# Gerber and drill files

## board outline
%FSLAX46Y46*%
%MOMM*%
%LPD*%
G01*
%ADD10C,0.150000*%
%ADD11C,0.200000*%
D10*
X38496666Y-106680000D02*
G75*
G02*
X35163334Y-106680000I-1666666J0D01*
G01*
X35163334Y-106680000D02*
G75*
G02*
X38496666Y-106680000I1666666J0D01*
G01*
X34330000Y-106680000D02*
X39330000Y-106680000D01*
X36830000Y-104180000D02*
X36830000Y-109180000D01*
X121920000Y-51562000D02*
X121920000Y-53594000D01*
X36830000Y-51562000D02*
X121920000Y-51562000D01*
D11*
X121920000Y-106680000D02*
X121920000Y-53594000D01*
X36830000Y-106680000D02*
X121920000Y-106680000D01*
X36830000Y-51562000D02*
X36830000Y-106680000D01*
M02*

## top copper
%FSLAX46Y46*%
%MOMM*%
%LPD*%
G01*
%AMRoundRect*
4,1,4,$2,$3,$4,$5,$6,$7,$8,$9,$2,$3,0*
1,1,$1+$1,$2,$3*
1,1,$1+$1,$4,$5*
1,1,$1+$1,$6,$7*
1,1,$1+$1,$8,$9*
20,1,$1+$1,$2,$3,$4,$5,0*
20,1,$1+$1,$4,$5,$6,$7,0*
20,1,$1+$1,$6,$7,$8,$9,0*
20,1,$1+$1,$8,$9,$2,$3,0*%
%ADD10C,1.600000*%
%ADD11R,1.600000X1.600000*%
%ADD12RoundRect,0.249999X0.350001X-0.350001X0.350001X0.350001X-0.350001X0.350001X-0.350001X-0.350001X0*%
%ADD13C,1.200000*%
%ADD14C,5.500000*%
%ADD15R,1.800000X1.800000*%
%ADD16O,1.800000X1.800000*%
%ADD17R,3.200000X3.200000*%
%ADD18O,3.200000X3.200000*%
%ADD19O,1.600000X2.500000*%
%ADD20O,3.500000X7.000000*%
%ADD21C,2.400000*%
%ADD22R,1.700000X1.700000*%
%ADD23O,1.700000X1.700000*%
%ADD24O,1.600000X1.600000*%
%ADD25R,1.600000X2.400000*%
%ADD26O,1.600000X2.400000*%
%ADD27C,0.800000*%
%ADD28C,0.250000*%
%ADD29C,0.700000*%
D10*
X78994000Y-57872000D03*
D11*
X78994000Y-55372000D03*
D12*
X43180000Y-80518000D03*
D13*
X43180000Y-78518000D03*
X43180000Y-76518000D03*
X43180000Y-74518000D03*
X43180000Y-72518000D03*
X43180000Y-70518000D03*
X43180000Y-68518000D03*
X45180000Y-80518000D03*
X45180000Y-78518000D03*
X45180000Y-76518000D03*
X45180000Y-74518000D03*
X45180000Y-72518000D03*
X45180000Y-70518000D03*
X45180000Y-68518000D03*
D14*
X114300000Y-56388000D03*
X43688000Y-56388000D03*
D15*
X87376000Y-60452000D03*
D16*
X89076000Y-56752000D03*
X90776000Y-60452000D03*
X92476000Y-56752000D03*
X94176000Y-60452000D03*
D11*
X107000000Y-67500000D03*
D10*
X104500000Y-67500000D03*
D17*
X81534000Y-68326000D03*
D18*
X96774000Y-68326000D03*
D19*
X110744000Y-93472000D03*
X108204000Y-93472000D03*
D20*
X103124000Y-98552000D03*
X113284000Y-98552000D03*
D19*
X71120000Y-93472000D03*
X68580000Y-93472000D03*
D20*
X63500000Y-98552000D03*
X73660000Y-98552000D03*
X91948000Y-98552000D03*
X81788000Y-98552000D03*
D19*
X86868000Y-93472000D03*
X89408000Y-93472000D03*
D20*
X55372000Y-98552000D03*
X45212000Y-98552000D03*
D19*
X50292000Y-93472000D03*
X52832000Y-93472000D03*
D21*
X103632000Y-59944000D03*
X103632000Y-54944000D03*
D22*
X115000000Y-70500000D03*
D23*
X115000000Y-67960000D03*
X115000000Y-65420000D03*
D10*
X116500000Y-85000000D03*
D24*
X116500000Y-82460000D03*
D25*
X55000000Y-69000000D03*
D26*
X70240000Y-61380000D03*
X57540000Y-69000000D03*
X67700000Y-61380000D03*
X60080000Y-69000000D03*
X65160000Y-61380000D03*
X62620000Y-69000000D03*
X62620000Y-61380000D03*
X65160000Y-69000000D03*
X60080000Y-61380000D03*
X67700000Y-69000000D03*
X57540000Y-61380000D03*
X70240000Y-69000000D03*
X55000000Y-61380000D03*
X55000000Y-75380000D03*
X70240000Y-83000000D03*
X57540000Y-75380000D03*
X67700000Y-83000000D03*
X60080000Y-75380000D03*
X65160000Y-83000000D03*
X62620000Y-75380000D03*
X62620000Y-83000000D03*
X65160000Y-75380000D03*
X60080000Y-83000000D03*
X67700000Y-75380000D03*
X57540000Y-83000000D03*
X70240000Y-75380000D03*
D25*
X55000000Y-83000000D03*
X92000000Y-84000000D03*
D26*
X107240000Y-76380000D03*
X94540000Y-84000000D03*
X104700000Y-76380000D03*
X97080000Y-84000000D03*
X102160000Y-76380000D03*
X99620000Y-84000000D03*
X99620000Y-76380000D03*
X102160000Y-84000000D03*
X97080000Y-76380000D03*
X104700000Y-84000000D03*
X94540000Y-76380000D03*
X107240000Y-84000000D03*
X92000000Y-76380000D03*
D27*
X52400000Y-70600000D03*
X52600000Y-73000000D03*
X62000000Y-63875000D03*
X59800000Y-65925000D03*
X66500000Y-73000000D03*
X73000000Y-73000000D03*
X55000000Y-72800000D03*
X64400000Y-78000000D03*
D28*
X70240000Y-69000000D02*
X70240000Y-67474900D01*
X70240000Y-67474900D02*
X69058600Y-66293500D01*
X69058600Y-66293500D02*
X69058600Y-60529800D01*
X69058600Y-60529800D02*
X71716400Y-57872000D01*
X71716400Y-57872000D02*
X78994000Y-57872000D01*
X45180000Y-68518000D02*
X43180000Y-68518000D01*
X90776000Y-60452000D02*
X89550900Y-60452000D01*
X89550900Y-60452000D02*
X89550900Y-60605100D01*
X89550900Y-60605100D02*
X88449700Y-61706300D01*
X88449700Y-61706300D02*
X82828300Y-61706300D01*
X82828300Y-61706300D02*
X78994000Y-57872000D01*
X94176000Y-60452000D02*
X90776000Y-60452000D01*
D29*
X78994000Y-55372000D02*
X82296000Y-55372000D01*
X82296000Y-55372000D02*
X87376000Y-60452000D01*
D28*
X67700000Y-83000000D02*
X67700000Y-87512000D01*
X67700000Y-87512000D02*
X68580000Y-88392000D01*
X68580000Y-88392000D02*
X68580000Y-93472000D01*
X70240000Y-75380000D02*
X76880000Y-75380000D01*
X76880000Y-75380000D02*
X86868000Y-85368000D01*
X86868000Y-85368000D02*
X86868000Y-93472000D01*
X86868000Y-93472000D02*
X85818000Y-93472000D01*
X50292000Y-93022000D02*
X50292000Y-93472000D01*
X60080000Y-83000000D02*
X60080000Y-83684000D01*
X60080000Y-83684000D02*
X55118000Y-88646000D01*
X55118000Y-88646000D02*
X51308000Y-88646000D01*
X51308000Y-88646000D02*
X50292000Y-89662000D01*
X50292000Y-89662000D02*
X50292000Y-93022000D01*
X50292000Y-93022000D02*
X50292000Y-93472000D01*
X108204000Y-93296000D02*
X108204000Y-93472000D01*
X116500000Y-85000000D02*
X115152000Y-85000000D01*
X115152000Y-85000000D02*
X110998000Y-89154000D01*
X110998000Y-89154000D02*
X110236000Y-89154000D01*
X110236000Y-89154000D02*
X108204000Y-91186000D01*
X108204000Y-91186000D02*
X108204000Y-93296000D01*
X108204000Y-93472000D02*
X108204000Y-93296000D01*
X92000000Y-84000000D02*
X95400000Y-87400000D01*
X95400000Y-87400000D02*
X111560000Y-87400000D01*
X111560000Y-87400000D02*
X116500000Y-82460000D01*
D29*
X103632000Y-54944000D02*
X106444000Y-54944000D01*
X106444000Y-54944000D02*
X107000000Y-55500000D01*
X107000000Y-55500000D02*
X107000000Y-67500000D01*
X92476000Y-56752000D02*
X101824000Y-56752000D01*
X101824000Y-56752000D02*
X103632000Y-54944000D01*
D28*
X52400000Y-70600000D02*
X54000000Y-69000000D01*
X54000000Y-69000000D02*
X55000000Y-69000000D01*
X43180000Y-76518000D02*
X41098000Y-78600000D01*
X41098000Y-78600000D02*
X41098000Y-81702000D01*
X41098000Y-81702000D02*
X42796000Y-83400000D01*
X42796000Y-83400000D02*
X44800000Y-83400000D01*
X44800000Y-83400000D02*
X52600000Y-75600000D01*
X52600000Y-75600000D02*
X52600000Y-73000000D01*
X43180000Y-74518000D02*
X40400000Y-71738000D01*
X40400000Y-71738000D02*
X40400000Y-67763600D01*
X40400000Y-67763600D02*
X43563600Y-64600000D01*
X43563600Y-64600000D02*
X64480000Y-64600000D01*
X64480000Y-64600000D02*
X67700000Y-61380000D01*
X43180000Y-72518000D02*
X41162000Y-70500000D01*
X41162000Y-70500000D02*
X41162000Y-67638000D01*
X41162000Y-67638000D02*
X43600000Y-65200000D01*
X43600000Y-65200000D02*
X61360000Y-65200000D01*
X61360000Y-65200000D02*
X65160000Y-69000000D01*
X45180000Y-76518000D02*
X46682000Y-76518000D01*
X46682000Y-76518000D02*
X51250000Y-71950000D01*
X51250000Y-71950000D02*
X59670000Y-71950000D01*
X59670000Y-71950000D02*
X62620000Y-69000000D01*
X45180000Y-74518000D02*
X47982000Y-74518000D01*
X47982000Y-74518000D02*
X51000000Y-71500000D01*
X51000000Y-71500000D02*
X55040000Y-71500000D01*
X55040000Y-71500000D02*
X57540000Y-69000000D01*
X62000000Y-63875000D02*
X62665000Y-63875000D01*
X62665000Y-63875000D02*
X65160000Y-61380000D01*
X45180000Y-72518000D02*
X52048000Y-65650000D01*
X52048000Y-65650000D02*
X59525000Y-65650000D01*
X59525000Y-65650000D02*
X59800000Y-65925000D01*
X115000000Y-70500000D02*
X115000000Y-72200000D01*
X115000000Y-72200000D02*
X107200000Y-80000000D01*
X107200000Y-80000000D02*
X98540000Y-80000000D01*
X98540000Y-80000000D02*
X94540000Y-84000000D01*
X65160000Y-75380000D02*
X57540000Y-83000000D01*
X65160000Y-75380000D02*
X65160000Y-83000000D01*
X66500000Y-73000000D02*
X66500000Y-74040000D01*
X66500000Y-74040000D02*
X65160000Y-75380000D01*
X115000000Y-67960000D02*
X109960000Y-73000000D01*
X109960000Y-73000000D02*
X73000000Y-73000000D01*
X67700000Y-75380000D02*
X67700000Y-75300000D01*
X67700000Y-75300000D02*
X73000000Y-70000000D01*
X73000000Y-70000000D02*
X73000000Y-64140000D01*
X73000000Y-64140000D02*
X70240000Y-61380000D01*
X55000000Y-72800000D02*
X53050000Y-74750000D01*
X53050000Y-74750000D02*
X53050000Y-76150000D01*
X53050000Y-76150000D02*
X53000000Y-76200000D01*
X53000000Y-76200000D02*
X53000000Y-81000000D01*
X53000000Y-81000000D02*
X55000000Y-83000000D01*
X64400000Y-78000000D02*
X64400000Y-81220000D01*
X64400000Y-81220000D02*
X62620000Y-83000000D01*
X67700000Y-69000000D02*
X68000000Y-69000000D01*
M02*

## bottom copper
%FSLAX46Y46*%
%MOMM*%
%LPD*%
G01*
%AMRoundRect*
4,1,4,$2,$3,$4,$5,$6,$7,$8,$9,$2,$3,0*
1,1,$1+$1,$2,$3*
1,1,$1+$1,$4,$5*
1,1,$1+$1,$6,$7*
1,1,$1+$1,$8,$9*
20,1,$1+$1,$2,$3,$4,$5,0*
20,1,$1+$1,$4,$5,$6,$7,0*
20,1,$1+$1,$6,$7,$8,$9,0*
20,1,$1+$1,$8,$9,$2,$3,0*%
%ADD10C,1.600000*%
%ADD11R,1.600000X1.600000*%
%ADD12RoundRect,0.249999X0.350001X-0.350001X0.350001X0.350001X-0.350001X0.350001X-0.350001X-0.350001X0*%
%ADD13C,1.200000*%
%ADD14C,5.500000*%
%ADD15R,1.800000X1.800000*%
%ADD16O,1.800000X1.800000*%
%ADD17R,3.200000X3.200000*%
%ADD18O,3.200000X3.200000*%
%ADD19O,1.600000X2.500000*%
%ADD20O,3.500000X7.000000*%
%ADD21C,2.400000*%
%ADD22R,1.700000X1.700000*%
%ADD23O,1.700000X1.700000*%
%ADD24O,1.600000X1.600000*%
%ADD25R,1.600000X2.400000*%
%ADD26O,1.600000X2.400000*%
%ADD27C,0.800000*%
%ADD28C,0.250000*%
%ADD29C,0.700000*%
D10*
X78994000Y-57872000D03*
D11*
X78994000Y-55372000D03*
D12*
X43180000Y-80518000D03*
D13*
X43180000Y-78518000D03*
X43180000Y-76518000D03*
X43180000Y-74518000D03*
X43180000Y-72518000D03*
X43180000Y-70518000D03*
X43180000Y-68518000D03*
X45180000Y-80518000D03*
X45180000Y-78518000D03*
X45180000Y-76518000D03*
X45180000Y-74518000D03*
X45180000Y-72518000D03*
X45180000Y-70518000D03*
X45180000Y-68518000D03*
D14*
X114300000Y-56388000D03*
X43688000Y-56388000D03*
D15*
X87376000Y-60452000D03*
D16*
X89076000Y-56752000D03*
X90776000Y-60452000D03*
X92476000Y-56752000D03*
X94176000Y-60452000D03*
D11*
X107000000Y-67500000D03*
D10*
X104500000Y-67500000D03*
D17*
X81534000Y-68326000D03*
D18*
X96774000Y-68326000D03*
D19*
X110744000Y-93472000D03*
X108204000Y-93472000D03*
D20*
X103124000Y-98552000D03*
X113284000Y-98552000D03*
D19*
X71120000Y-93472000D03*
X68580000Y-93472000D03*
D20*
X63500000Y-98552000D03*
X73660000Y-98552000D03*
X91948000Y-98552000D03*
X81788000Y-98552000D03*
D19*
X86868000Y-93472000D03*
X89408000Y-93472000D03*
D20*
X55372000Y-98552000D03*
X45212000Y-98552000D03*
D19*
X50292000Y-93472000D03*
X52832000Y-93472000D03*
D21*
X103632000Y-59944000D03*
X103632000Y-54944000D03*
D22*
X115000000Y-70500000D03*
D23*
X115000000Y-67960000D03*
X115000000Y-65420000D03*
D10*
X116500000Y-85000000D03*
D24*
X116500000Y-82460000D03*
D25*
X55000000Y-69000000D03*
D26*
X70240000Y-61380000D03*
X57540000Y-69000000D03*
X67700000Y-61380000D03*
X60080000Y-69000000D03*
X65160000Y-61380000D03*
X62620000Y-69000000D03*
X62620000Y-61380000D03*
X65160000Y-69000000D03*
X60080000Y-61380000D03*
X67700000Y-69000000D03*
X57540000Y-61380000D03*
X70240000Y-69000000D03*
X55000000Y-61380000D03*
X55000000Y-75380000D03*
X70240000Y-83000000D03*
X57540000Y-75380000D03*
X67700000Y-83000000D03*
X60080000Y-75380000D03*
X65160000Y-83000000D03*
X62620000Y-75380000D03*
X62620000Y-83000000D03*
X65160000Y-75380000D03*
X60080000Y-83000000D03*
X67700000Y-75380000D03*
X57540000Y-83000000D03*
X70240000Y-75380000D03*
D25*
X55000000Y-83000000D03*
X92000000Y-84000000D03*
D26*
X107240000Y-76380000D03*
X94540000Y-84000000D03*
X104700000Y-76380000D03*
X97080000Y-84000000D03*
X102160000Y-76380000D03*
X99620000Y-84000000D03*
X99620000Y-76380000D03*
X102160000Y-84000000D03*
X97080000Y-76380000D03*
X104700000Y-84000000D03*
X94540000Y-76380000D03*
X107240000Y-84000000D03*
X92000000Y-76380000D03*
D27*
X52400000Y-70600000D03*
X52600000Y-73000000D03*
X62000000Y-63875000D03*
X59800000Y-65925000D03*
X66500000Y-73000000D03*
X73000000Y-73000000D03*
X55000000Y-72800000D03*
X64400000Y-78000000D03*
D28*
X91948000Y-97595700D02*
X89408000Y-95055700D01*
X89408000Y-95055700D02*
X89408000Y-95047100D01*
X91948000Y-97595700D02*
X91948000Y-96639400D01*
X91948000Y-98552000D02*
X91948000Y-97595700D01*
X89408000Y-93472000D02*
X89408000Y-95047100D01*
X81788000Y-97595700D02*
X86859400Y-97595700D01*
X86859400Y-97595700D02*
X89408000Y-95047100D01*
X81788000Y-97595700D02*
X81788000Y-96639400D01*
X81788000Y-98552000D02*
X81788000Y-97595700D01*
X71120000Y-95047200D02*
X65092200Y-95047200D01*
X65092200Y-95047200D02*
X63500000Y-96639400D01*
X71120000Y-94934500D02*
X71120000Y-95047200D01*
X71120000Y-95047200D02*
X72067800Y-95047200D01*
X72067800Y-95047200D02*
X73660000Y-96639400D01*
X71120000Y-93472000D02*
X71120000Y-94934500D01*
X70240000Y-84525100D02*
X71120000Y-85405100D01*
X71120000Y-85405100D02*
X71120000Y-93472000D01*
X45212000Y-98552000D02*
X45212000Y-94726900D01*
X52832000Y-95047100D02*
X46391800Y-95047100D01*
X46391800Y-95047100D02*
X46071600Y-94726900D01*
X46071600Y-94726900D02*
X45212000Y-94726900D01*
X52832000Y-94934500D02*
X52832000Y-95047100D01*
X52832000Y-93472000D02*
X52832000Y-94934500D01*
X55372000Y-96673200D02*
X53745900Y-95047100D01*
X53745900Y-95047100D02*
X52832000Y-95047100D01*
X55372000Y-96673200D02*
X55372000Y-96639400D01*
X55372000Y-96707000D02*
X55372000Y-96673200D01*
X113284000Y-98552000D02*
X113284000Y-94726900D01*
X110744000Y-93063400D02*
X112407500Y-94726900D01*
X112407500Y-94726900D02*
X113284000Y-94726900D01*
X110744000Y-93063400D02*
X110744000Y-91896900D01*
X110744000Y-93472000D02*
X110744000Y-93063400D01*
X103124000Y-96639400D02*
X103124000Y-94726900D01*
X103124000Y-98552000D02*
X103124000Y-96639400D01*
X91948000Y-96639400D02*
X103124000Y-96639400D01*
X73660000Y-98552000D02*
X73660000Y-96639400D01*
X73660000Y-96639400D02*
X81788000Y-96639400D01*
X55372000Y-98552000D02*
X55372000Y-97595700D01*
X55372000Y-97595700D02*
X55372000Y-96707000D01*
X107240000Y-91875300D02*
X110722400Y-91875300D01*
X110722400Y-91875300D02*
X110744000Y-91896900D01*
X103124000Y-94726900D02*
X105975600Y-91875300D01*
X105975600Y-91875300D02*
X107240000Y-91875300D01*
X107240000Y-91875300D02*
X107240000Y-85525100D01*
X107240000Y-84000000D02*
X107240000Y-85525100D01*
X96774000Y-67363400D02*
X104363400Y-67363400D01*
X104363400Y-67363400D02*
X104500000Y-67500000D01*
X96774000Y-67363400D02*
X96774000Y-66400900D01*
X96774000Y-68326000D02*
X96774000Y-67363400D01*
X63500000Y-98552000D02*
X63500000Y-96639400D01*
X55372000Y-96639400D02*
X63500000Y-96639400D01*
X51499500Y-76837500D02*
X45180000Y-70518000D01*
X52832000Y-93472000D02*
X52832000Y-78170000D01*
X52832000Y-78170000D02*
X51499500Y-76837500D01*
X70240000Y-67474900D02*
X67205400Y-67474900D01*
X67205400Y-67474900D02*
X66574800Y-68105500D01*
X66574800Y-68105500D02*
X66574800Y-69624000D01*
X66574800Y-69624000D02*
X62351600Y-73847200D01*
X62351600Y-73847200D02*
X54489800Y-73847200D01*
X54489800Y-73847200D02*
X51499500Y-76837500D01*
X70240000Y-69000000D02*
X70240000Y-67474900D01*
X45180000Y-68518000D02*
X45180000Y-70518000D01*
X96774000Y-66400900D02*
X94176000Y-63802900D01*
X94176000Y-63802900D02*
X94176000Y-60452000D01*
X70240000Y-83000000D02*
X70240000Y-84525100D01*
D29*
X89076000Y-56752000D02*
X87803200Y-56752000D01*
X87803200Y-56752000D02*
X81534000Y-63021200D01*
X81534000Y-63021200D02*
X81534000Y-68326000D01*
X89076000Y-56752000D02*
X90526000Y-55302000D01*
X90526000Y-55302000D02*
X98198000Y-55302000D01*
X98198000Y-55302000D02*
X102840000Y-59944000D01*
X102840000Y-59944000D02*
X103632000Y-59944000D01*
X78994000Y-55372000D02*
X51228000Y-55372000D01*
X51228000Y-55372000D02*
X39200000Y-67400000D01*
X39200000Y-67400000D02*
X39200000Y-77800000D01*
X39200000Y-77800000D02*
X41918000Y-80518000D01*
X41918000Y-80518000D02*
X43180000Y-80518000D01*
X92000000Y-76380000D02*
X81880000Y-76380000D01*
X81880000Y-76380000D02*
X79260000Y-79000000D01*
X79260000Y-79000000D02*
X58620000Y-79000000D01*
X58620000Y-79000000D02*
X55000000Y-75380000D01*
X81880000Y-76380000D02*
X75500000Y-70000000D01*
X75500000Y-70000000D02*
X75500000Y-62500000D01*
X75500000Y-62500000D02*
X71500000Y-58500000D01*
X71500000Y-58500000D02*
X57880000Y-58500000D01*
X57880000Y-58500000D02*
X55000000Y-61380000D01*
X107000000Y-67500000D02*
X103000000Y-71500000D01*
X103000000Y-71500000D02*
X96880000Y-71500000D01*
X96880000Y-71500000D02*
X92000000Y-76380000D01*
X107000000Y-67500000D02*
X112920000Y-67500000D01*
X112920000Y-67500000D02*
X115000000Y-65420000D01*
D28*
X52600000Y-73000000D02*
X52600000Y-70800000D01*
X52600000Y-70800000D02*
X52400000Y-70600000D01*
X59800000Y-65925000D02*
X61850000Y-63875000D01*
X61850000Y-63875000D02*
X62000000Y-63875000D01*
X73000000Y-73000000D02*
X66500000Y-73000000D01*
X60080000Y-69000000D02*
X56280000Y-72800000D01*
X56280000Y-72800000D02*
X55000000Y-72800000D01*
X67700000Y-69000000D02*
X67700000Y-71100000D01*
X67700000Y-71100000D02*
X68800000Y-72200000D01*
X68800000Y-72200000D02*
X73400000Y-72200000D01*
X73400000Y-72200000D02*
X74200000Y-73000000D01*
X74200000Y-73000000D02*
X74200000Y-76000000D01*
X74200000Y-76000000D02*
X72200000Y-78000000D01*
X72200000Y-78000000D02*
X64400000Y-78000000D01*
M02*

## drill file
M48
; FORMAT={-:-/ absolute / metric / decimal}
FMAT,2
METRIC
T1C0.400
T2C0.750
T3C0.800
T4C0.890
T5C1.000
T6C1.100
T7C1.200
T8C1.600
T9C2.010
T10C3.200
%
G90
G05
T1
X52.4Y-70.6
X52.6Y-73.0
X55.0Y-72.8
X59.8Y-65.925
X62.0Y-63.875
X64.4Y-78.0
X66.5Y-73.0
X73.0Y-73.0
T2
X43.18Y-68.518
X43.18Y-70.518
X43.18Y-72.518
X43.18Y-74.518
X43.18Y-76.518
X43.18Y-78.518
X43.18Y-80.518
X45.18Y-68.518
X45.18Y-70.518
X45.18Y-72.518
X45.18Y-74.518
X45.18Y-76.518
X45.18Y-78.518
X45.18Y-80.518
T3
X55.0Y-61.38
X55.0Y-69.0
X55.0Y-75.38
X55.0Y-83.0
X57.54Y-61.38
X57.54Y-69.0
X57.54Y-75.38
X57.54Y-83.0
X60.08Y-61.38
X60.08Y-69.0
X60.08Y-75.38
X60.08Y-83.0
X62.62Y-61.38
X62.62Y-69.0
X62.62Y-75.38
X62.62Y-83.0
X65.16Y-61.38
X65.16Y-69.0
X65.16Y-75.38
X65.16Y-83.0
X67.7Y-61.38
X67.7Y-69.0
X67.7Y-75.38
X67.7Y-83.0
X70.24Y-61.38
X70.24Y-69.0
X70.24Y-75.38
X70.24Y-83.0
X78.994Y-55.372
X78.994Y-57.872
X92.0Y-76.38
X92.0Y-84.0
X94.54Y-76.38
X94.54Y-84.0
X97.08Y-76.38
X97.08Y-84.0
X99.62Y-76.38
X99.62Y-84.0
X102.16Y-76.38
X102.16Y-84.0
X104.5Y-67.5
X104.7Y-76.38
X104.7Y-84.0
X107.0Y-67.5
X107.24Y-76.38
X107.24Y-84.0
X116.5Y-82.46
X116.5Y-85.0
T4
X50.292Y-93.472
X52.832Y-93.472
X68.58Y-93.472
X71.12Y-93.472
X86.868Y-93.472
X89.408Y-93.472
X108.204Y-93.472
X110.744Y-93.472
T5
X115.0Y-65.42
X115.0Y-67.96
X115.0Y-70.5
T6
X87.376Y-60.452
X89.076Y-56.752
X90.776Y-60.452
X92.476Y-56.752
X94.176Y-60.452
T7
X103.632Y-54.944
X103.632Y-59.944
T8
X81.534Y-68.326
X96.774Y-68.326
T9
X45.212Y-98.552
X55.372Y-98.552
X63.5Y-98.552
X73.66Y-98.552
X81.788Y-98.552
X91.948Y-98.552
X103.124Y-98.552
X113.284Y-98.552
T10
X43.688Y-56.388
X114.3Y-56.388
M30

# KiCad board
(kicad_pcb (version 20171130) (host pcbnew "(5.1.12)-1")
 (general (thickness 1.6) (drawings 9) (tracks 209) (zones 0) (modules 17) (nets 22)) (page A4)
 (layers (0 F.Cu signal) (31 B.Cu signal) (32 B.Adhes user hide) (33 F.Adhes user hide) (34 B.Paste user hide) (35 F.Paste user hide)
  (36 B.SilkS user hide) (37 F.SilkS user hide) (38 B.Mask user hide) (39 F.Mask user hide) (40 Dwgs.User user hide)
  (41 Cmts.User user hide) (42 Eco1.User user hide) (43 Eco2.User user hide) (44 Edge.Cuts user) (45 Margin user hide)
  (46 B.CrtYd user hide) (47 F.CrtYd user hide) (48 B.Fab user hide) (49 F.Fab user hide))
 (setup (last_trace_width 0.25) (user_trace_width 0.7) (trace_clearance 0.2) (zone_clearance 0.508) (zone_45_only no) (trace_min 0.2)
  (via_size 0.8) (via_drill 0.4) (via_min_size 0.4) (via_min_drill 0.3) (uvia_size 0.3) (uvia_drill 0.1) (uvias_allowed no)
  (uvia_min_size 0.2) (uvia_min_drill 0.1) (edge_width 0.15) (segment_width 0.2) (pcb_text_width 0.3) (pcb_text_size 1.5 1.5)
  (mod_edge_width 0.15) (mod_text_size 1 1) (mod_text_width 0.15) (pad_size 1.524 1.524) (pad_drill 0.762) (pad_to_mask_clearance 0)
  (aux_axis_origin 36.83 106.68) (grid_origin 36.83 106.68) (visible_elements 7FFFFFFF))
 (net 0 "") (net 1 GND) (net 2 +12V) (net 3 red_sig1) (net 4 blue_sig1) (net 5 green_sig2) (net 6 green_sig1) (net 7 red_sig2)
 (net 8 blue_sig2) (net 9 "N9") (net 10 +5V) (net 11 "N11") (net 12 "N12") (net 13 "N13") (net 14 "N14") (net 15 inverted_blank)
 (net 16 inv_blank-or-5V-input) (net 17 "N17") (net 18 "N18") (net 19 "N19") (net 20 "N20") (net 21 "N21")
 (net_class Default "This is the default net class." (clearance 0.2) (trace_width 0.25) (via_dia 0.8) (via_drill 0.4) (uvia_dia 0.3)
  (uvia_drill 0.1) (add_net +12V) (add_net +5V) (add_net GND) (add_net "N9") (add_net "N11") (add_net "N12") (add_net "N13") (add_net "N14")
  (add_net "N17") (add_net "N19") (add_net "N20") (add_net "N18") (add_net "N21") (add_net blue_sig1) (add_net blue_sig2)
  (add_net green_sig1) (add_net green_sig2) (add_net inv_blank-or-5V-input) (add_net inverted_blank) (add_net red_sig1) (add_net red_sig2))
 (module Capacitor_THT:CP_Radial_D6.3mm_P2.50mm (layer F.Cu) (at 78.994 55.372 270)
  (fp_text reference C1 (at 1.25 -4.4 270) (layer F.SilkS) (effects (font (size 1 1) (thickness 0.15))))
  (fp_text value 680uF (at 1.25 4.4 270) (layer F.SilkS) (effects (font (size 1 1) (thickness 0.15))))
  (pad 2 thru_hole circle (at 2.5 0 270) (size 1.6 1.6) (drill 0.8) (layers *.Cu *.Mask) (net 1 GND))
  (pad 1 thru_hole rect (at 0 0 270) (size 1.6 1.6) (drill 0.8) (layers *.Cu *.Mask) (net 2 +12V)))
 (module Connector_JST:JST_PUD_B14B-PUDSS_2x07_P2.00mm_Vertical (layer F.Cu) (at 43.18 80.518 90)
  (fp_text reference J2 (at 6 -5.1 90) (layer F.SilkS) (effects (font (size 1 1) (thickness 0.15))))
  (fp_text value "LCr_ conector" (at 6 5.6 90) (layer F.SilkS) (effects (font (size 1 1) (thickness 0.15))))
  (pad 1 thru_hole roundrect (at 0 0 90) (size 1.2 1.2) (drill 0.75) (layers *.Cu *.Mask) (roundrect_rratio 0.2083325) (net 2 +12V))
  (pad 3 thru_hole circle (at 2 0 90) (size 1.2 1.2) (drill 0.75) (layers *.Cu *.Mask))
  (pad 5 thru_hole circle (at 4 0 90) (size 1.2 1.2) (drill 0.75) (layers *.Cu *.Mask) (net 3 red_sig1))
  (pad 7 thru_hole circle (at 6 0 90) (size 1.2 1.2) (drill 0.75) (layers *.Cu *.Mask) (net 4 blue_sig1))
  (pad 9 thru_hole circle (at 8 0 90) (size 1.2 1.2) (drill 0.75) (layers *.Cu *.Mask) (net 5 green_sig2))
  (pad 11 thru_hole circle (at 10 0 90) (size 1.2 1.2) (drill 0.75) (layers *.Cu *.Mask))
  (pad 13 thru_hole circle (at 12 0 90) (size 1.2 1.2) (drill 0.75) (layers *.Cu *.Mask) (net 1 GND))
  (pad 2 thru_hole circle (at 0 2 90) (size 1.2 1.2) (drill 0.75) (layers *.Cu *.Mask))
  (pad 4 thru_hole circle (at 2 2 90) (size 1.2 1.2) (drill 0.75) (layers *.Cu *.Mask))
  (pad 6 thru_hole circle (at 4 2 90) (size 1.2 1.2) (drill 0.75) (layers *.Cu *.Mask) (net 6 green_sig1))
  (pad 8 thru_hole circle (at 6 2 90) (size 1.2 1.2) (drill 0.75) (layers *.Cu *.Mask) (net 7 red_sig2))
  (pad 10 thru_hole circle (at 8 2 90) (size 1.2 1.2) (drill 0.75) (layers *.Cu *.Mask) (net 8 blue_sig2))
  (pad 12 thru_hole circle (at 10 2 90) (size 1.2 1.2) (drill 0.75) (layers *.Cu *.Mask) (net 1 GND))
  (pad 14 thru_hole circle (at 12 2 90) (size 1.2 1.2) (drill 0.75) (layers *.Cu *.Mask) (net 1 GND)))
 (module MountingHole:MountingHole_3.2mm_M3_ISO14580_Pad (layer F.Cu) (at 114.3 56.388)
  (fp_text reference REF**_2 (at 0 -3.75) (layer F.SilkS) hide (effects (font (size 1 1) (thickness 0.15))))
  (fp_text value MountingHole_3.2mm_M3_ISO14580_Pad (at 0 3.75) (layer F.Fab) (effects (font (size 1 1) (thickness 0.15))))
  (pad 1 thru_hole circle (at 0 0) (size 5.5 5.5) (drill 3.2) (layers *.Cu *.Mask)))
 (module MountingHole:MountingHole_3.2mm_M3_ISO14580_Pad (layer F.Cu) (at 43.688 56.388)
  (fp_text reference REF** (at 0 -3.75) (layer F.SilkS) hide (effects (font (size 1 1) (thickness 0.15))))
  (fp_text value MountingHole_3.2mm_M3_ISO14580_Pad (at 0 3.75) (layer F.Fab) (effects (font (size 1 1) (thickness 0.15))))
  (pad 1 thru_hole circle (at 0 0) (size 5.5 5.5) (drill 3.2) (layers *.Cu *.Mask)))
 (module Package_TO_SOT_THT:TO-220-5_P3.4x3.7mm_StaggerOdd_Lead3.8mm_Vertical (layer F.Cu) (at 87.376 60.452)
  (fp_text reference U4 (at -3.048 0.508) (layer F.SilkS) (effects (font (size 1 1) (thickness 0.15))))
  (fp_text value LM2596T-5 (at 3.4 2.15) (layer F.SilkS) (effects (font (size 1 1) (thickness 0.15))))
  (pad 1 thru_hole rect (at 0 0) (size 1.8 1.8) (drill 1.1) (layers *.Cu *.Mask) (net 2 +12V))
  (pad 2 thru_hole oval (at 1.7 -3.7) (size 1.8 1.8) (drill 1.1) (layers *.Cu *.Mask) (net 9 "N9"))
  (pad 3 thru_hole oval (at 3.4 0) (size 1.8 1.8) (drill 1.1) (layers *.Cu *.Mask) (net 1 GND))
  (pad 4 thru_hole oval (at 5.1 -3.7) (size 1.8 1.8) (drill 1.1) (layers *.Cu *.Mask) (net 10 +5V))
  (pad 5 thru_hole oval (at 6.8 0) (size 1.8 1.8) (drill 1.1) (layers *.Cu *.Mask) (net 1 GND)))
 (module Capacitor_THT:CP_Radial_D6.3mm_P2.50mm (layer F.Cu) (at 107 67.5 180)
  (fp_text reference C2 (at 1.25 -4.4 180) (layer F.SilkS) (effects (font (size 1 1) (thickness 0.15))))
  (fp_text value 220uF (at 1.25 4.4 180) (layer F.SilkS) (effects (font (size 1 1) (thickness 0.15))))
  (pad 1 thru_hole rect (at 0 0 180) (size 1.6 1.6) (drill 0.8) (layers *.Cu *.Mask) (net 10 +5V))
  (pad 2 thru_hole circle (at 2.5 0 180) (size 1.6 1.6) (drill 0.8) (layers *.Cu *.Mask) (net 1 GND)))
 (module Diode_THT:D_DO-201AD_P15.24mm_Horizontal (layer F.Cu) (at 81.534 68.326)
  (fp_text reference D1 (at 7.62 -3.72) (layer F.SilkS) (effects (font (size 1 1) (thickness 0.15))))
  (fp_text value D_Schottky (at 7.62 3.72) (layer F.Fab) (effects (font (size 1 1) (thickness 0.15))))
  (pad 1 thru_hole rect (at 0 0) (size 3.2 3.2) (drill 1.6) (layers *.Cu *.Mask) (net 9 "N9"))
  (pad 2 thru_hole oval (at 15.24 0) (size 3.2 3.2) (drill 1.6) (layers *.Cu *.Mask) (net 1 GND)))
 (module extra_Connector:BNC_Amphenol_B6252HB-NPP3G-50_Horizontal (layer F.Cu) (at 108.204 93.472 180)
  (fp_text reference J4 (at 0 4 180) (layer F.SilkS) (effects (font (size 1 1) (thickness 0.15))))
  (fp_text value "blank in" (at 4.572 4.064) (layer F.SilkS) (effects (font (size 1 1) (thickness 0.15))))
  (pad 2 thru_hole oval (at -2.54 0 180) (size 1.6 2.5) (drill 0.89) (layers *.Cu *.Mask) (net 1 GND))
  (pad 1 thru_hole oval (at 0 0 180) (size 1.6 2.5) (drill 0.89) (layers *.Cu *.Mask) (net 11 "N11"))
  (pad 2 thru_hole oval (at 5.08 -5.08 180) (size 3.5 7) (drill 2.01) (layers *.Cu *.Mask) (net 1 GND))
  (pad 2 thru_hole oval (at -5.08 -5.08 180) (size 3.5 7) (drill 2.01) (layers *.Cu *.Mask) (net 1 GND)))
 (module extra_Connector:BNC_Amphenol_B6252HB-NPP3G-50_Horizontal (layer F.Cu) (at 68.58 93.472 180)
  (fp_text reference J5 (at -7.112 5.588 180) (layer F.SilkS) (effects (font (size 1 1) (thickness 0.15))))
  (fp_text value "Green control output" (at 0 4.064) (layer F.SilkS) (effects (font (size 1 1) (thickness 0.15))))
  (pad 2 thru_hole oval (at -2.54 0 180) (size 1.6 2.5) (drill 0.89) (layers *.Cu *.Mask) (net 1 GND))
  (pad 1 thru_hole oval (at 0 0 180) (size 1.6 2.5) (drill 0.89) (layers *.Cu *.Mask) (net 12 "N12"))
  (pad 2 thru_hole oval (at 5.08 -5.08 180) (size 3.5 7) (drill 2.01) (layers *.Cu *.Mask) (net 1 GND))
  (pad 2 thru_hole oval (at -5.08 -5.08 180) (size 3.5 7) (drill 2.01) (layers *.Cu *.Mask) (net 1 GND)))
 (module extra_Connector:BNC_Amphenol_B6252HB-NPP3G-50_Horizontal (layer F.Cu) (at 86.868 93.472 180)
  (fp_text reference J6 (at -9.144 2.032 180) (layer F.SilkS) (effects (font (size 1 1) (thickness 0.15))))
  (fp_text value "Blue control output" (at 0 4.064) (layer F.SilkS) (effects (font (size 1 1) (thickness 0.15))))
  (pad 2 thru_hole oval (at -5.08 -5.08 180) (size 3.5 7) (drill 2.01) (layers *.Cu *.Mask) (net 1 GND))
  (pad 2 thru_hole oval (at 5.08 -5.08 180) (size 3.5 7) (drill 2.01) (layers *.Cu *.Mask) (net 1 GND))
  (pad 1 thru_hole oval (at 0 0 180) (size 1.6 2.5) (drill 0.89) (layers *.Cu *.Mask) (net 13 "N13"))
  (pad 2 thru_hole oval (at -2.54 0 180) (size 1.6 2.5) (drill 0.89) (layers *.Cu *.Mask) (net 1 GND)))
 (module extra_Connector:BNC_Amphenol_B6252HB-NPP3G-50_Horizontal (layer F.Cu) (at 50.292 93.472 180)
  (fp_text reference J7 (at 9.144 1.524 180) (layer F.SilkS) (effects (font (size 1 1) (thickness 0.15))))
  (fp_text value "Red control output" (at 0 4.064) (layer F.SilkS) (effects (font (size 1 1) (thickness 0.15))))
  (pad 2 thru_hole oval (at -5.08 -5.08 180) (size 3.5 7) (drill 2.01) (layers *.Cu *.Mask) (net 1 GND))
  (pad 2 thru_hole oval (at 5.08 -5.08 180) (size 3.5 7) (drill 2.01) (layers *.Cu *.Mask) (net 1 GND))
  (pad 1 thru_hole oval (at 0 0 180) (size 1.6 2.5) (drill 0.89) (layers *.Cu *.Mask) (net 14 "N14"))
  (pad 2 thru_hole oval (at -2.54 0 180) (size 1.6 2.5) (drill 0.89) (layers *.Cu *.Mask) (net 1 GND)))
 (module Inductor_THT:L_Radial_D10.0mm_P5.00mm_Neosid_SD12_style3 (layer F.Cu) (at 103.632 59.944 90)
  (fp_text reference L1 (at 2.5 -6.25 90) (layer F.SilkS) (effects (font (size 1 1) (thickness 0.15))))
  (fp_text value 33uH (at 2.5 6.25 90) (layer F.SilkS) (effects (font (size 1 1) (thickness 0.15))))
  (pad 1 thru_hole circle (at 0 0 90) (size 2.4 2.4) (drill 1.2) (layers *.Cu *.Mask) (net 9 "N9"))
  (pad 2 thru_hole circle (at 5 0 90) (size 2.4 2.4) (drill 1.2) (layers *.Cu *.Mask) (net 10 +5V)))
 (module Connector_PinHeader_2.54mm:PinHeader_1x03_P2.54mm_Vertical (layer F.Cu) (at 115 70.5 180)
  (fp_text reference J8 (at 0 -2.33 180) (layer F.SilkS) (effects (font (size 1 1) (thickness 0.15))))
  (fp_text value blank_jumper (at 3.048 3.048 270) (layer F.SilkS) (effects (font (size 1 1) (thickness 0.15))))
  (pad 1 thru_hole rect (at 0 0 180) (size 1.7 1.7) (drill 1) (layers *.Cu *.Mask) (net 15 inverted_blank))
  (pad 2 thru_hole oval (at 0 2.54 180) (size 1.7 1.7) (drill 1) (layers *.Cu *.Mask) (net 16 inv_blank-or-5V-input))
  (pad 3 thru_hole oval (at 0 5.08 180) (size 1.7 1.7) (drill 1) (layers *.Cu *.Mask) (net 10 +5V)))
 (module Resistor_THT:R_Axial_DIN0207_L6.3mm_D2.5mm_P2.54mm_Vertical (layer F.Cu) (at 116.5 85 90)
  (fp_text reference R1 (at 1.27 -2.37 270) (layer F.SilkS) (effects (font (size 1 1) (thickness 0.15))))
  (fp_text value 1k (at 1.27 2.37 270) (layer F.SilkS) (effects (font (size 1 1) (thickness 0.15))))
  (pad 1 thru_hole circle (at 0 0 90) (size 1.6 1.6) (drill 0.8) (layers *.Cu *.Mask) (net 11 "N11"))
  (pad 2 thru_hole oval (at 2.54 0 90) (size 1.6 1.6) (drill 0.8) (layers *.Cu *.Mask) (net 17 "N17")))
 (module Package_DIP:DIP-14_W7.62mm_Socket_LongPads (layer F.Cu) (at 55 69 90)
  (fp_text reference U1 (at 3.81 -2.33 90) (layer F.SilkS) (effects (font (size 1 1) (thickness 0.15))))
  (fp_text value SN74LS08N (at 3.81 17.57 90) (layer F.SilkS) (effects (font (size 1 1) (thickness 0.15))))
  (pad 1 thru_hole rect (at 0 0 90) (size 2.4 1.6) (drill 0.8) (layers *.Cu *.Mask) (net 3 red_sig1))
  (pad 8 thru_hole oval (at 7.62 15.24 90) (size 2.4 1.6) (drill 0.8) (layers *.Cu *.Mask) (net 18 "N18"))
  (pad 2 thru_hole oval (at 0 2.54 90) (size 2.4 1.6) (drill 0.8) (layers *.Cu *.Mask) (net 7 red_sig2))
  (pad 9 thru_hole oval (at 7.62 12.7 90) (size 2.4 1.6) (drill 0.8) (layers *.Cu *.Mask) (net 4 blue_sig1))
  (pad 3 thru_hole oval (at 0 5.08 90) (size 2.4 1.6) (drill 0.8) (layers *.Cu *.Mask) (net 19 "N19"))
  (pad 10 thru_hole oval (at 7.62 10.16 90) (size 2.4 1.6) (drill 0.8) (layers *.Cu *.Mask) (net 8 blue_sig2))
  (pad 4 thru_hole oval (at 0 7.62 90) (size 2.4 1.6) (drill 0.8) (layers *.Cu *.Mask) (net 6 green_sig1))
  (pad 11 thru_hole oval (at 7.62 7.62 90) (size 2.4 1.6) (drill 0.8) (layers *.Cu *.Mask))
  (pad 5 thru_hole oval (at 0 10.16 90) (size 2.4 1.6) (drill 0.8) (layers *.Cu *.Mask) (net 5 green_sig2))
  (pad 12 thru_hole oval (at 7.62 5.08 90) (size 2.4 1.6) (drill 0.8) (layers *.Cu *.Mask))
  (pad 6 thru_hole oval (at 0 12.7 90) (size 2.4 1.6) (drill 0.8) (layers *.Cu *.Mask) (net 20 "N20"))
  (pad 13 thru_hole oval (at 7.62 2.54 90) (size 2.4 1.6) (drill 0.8) (layers *.Cu *.Mask))
  (pad 7 thru_hole oval (at 0 15.24 90) (size 2.4 1.6) (drill 0.8) (layers *.Cu *.Mask) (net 1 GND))
  (pad 14 thru_hole oval (at 7.62 0 90) (size 2.4 1.6) (drill 0.8) (layers *.Cu *.Mask) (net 10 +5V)))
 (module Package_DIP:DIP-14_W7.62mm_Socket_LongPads (layer F.Cu) (at 55 83 90)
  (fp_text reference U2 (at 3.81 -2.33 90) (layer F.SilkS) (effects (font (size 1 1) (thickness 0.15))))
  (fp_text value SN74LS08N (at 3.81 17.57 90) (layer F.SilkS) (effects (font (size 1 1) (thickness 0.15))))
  (pad 14 thru_hole oval (at 7.62 0 90) (size 2.4 1.6) (drill 0.8) (layers *.Cu *.Mask) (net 10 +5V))
  (pad 7 thru_hole oval (at 0 15.24 90) (size 2.4 1.6) (drill 0.8) (layers *.Cu *.Mask) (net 1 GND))
  (pad 13 thru_hole oval (at 7.62 2.54 90) (size 2.4 1.6) (drill 0.8) (layers *.Cu *.Mask))
  (pad 6 thru_hole oval (at 0 12.7 90) (size 2.4 1.6) (drill 0.8) (layers *.Cu *.Mask) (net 12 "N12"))
  (pad 12 thru_hole oval (at 7.62 5.08 90) (size 2.4 1.6) (drill 0.8) (layers *.Cu *.Mask))
  (pad 5 thru_hole oval (at 0 10.16 90) (size 2.4 1.6) (drill 0.8) (layers *.Cu *.Mask) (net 16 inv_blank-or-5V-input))
  (pad 11 thru_hole oval (at 7.62 7.62 90) (size 2.4 1.6) (drill 0.8) (layers *.Cu *.Mask))
  (pad 4 thru_hole oval (at 0 7.62 90) (size 2.4 1.6) (drill 0.8) (layers *.Cu *.Mask) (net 20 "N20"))
  (pad 10 thru_hole oval (at 7.62 10.16 90) (size 2.4 1.6) (drill 0.8) (layers *.Cu *.Mask) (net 16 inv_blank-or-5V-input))
  (pad 3 thru_hole oval (at 0 5.08 90) (size 2.4 1.6) (drill 0.8) (layers *.Cu *.Mask) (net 14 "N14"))
  (pad 9 thru_hole oval (at 7.62 12.7 90) (size 2.4 1.6) (drill 0.8) (layers *.Cu *.Mask) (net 18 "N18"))
  (pad 2 thru_hole oval (at 0 2.54 90) (size 2.4 1.6) (drill 0.8) (layers *.Cu *.Mask) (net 16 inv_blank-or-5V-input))
  (pad 8 thru_hole oval (at 7.62 15.24 90) (size 2.4 1.6) (drill 0.8) (layers *.Cu *.Mask) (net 13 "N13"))
  (pad 1 thru_hole rect (at 0 0 90) (size 2.4 1.6) (drill 0.8) (layers *.Cu *.Mask) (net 19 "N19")))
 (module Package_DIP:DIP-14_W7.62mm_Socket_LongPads (layer F.Cu) (at 92 84 90)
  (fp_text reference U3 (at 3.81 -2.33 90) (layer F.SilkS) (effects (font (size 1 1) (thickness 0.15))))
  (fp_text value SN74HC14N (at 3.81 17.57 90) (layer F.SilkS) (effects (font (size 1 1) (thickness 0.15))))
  (pad 1 thru_hole rect (at 0 0 90) (size 2.4 1.6) (drill 0.8) (layers *.Cu *.Mask) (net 17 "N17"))
  (pad 8 thru_hole oval (at 7.62 15.24 90) (size 2.4 1.6) (drill 0.8) (layers *.Cu *.Mask))
  (pad 2 thru_hole oval (at 0 2.54 90) (size 2.4 1.6) (drill 0.8) (layers *.Cu *.Mask) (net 15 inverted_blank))
  (pad 9 thru_hole oval (at 7.62 12.7 90) (size 2.4 1.6) (drill 0.8) (layers *.Cu *.Mask))
  (pad 3 thru_hole oval (at 0 5.08 90) (size 2.4 1.6) (drill 0.8) (layers *.Cu *.Mask))
  (pad 10 thru_hole oval (at 7.62 10.16 90) (size 2.4 1.6) (drill 0.8) (layers *.Cu *.Mask))
  (pad 4 thru_hole oval (at 0 7.62 90) (size 2.4 1.6) (drill 0.8) (layers *.Cu *.Mask) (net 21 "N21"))
  (pad 11 thru_hole oval (at 7.62 7.62 90) (size 2.4 1.6) (drill 0.8) (layers *.Cu *.Mask))
  (pad 5 thru_hole oval (at 0 10.16 90) (size 2.4 1.6) (drill 0.8) (layers *.Cu *.Mask))
  (pad 12 thru_hole oval (at 7.62 5.08 90) (size 2.4 1.6) (drill 0.8) (layers *.Cu *.Mask))
  (pad 6 thru_hole oval (at 0 12.7 90) (size 2.4 1.6) (drill 0.8) (layers *.Cu *.Mask))
  (pad 13 thru_hole oval (at 7.62 2.54 90) (size 2.4 1.6) (drill 0.8) (layers *.Cu *.Mask))
  (pad 7 thru_hole oval (at 0 15.24 90) (size 2.4 1.6) (drill 0.8) (layers *.Cu *.Mask) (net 1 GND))
  (pad 14 thru_hole oval (at 7.62 0 90) (size 2.4 1.6) (drill 0.8) (layers *.Cu *.Mask) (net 10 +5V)))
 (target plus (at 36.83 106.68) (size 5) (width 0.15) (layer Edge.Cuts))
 (gr_line (start 121.92 51.562) (end 121.92 53.594) (layer Edge.Cuts) (width 0.15))
 (gr_line (start 36.83 51.562) (end 121.92 51.562) (layer Edge.Cuts) (width 0.15))
 (gr_line (start 121.92 106.68) (end 121.92 53.594) (layer Edge.Cuts) (width 0.2))
 (gr_line (start 36.83 106.68) (end 121.92 106.68) (layer Edge.Cuts) (width 0.2))
 (gr_line (start 36.83 51.562) (end 36.83 106.68) (layer Edge.Cuts) (width 0.2))
 (segment (start 91.948 97.5957) (end 89.408 95.0557) (width 0.25) (layer B.Cu) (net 1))
 (segment (start 89.408 95.0557) (end 89.408 95.0471) (width 0.25) (layer B.Cu) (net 1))
 (segment (start 91.948 97.5957) (end 91.948 96.6394) (width 0.25) (layer B.Cu) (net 1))
 (segment (start 91.948 98.552) (end 91.948 97.5957) (width 0.25) (layer B.Cu) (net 1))
 (segment (start 89.408 93.472) (end 89.408 95.0471) (width 0.25) (layer B.Cu) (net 1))
 (segment (start 81.788 97.5957) (end 86.8594 97.5957) (width 0.25) (layer B.Cu) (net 1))
 (segment (start 86.8594 97.5957) (end 89.408 95.0471) (width 0.25) (layer B.Cu) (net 1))
 (segment (start 81.788 97.5957) (end 81.788 96.6394) (width 0.25) (layer B.Cu) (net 1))
 (segment (start 81.788 98.552) (end 81.788 97.5957) (width 0.25) (layer B.Cu) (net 1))
 (segment (start 70.24 69) (end 70.24 67.4749) (width 0.25) (layer F.Cu) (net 1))
 (segment (start 70.24 67.4749) (end 69.0586 66.2935) (width 0.25) (layer F.Cu) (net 1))
 (segment (start 69.0586 66.2935) (end 69.0586 60.5298) (width 0.25) (layer F.Cu) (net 1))
 (segment (start 69.0586 60.5298) (end 71.7164 57.872) (width 0.25) (layer F.Cu) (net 1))
 (segment (start 71.7164 57.872) (end 78.994 57.872) (width 0.25) (layer F.Cu) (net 1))
 (segment (start 71.12 95.0472) (end 65.0922 95.0472) (width 0.25) (layer B.Cu) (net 1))
 (segment (start 65.0922 95.0472) (end 63.5 96.6394) (width 0.25) (layer B.Cu) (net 1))
 (segment (start 71.12 94.9345) (end 71.12 95.0472) (width 0.25) (layer B.Cu) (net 1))
 (segment (start 71.12 95.0472) (end 72.0678 95.0472) (width 0.25) (layer B.Cu) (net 1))
 (segment (start 72.0678 95.0472) (end 73.66 96.6394) (width 0.25) (layer B.Cu) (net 1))
 (segment (start 71.12 93.472) (end 71.12 94.9345) (width 0.25) (layer B.Cu) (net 1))
 (segment (start 70.24 84.5251) (end 71.12 85.4051) (width 0.25) (layer B.Cu) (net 1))
 (segment (start 71.12 85.4051) (end 71.12 93.472) (width 0.25) (layer B.Cu) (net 1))
 (segment (start 45.212 98.552) (end 45.212 94.7269) (width 0.25) (layer B.Cu) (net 1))
 (segment (start 52.832 95.0471) (end 46.3918 95.0471) (width 0.25) (layer B.Cu) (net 1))
 (segment (start 46.3918 95.0471) (end 46.0716 94.7269) (width 0.25) (layer B.Cu) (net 1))
 (segment (start 46.0716 94.7269) (end 45.212 94.7269) (width 0.25) (layer B.Cu) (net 1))
 (segment (start 52.832 94.9345) (end 52.832 95.0471) (width 0.25) (layer B.Cu) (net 1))
 (segment (start 52.832 93.472) (end 52.832 94.9345) (width 0.25) (layer B.Cu) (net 1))
 (segment (start 55.372 96.6732) (end 53.7459 95.0471) (width 0.25) (layer B.Cu) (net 1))
 (segment (start 53.7459 95.0471) (end 52.832 95.0471) (width 0.25) (layer B.Cu) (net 1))
 (segment (start 55.372 96.6732) (end 55.372 96.6394) (width 0.25) (layer B.Cu) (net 1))
 (segment (start 55.372 96.707) (end 55.372 96.6732) (width 0.25) (layer B.Cu) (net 1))
 (segment (start 113.284 98.552) (end 113.284 94.7269) (width 0.25) (layer B.Cu) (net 1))
 (segment (start 110.744 93.0634) (end 112.4075 94.7269) (width 0.25) (layer B.Cu) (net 1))
 (segment (start 112.4075 94.7269) (end 113.284 94.7269) (width 0.25) (layer B.Cu) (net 1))
 (segment (start 110.744 93.0634) (end 110.744 91.8969) (width 0.25) (layer B.Cu) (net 1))
 (segment (start 110.744 93.472) (end 110.744 93.0634) (width 0.25) (layer B.Cu) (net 1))
 (segment (start 103.124 96.6394) (end 103.124 94.7269) (width 0.25) (layer B.Cu) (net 1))
 (segment (start 103.124 98.552) (end 103.124 96.6394) (width 0.25) (layer B.Cu) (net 1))
 (segment (start 91.948 96.6394) (end 103.124 96.6394) (width 0.25) (layer B.Cu) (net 1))
 (segment (start 73.66 98.552) (end 73.66 96.6394) (width 0.25) (layer B.Cu) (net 1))
 (segment (start 73.66 96.6394) (end 81.788 96.6394) (width 0.25) (layer B.Cu) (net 1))
 (segment (start 55.372 98.552) (end 55.372 97.5957) (width 0.25) (layer B.Cu) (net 1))
 (segment (start 55.372 97.5957) (end 55.372 96.707) (width 0.25) (layer B.Cu) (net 1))
 (segment (start 107.24 91.8753) (end 110.7224 91.8753) (width 0.25) (layer B.Cu) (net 1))
 (segment (start 110.7224 91.8753) (end 110.744 91.8969) (width 0.25) (layer B.Cu) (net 1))
 (segment (start 103.124 94.7269) (end 105.9756 91.8753) (width 0.25) (layer B.Cu) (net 1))
 (segment (start 105.9756 91.8753) (end 107.24 91.8753) (width 0.25) (layer B.Cu) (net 1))
 (segment (start 107.24 91.8753) (end 107.24 85.5251) (width 0.25) (layer B.Cu) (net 1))
 (segment (start 107.24 84) (end 107.24 85.5251) (width 0.25) (layer B.Cu) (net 1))
 (segment (start 96.774 67.3634) (end 104.3634 67.3634) (width 0.25) (layer B.Cu) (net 1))
 (segment (start 104.3634 67.3634) (end 104.5 67.5) (width 0.25) (layer B.Cu) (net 1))
 (segment (start 96.774 67.3634) (end 96.774 66.4009) (width 0.25) (layer B.Cu) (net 1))
 (segment (start 96.774 68.326) (end 96.774 67.3634) (width 0.25) (layer B.Cu) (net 1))
 (segment (start 63.5 98.552) (end 63.5 96.6394) (width 0.25) (layer B.Cu) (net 1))
 (segment (start 55.372 96.6394) (end 63.5 96.6394) (width 0.25) (layer B.Cu) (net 1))
 (segment (start 51.4995 76.8375) (end 45.18 70.518) (width 0.25) (layer B.Cu) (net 1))
 (segment (start 52.832 93.472) (end 52.832 78.17) (width 0.25) (layer B.Cu) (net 1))
 (segment (start 52.832 78.17) (end 51.4995 76.8375) (width 0.25) (layer B.Cu) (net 1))
 (segment (start 70.24 67.4749) (end 67.2054 67.4749) (width 0.25) (layer B.Cu) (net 1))
 (segment (start 67.2054 67.4749) (end 66.5748 68.1055) (width 0.25) (layer B.Cu) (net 1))
 (segment (start 66.5748 68.1055) (end 66.5748 69.624) (width 0.25) (layer B.Cu) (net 1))
 (segment (start 66.5748 69.624) (end 62.3516 73.8472) (width 0.25) (layer B.Cu) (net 1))
 (segment (start 62.3516 73.8472) (end 54.4898 73.8472) (width 0.25) (layer B.Cu) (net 1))
 (segment (start 54.4898 73.8472) (end 51.4995 76.8375) (width 0.25) (layer B.Cu) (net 1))
 (segment (start 70.24 69) (end 70.24 67.4749) (width 0.25) (layer B.Cu) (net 1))
 (segment (start 45.18 68.518) (end 43.18 68.518) (width 0.25) (layer F.Cu) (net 1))
 (segment (start 45.18 68.518) (end 45.18 70.518) (width 0.25) (layer B.Cu) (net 1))
 (segment (start 90.776 60.452) (end 89.5509 60.452) (width 0.25) (layer F.Cu) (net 1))
 (segment (start 89.5509 60.452) (end 89.5509 60.6051) (width 0.25) (layer F.Cu) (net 1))
 (segment (start 89.5509 60.6051) (end 88.4497 61.7063) (width 0.25) (layer F.Cu) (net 1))
 (segment (start 88.4497 61.7063) (end 82.8283 61.7063) (width 0.25) (layer F.Cu) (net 1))
 (segment (start 82.8283 61.7063) (end 78.994 57.872) (width 0.25) (layer F.Cu) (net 1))
 (segment (start 94.176 60.452) (end 90.776 60.452) (width 0.25) (layer F.Cu) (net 1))
 (segment (start 96.774 66.4009) (end 94.176 63.8029) (width 0.25) (layer B.Cu) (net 1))
 (segment (start 94.176 63.8029) (end 94.176 60.452) (width 0.25) (layer B.Cu) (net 1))
 (segment (start 70.24 83) (end 70.24 84.5251) (width 0.25) (layer B.Cu) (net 1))
 (segment (start 89.076 56.752) (end 87.8032 56.752) (width 0.7) (layer B.Cu) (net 9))
 (segment (start 87.8032 56.752) (end 81.534 63.0212) (width 0.7) (layer B.Cu) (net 9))
 (segment (start 81.534 63.0212) (end 81.534 68.326) (width 0.7) (layer B.Cu) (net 9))
 (segment (start 89.076 56.752) (end 90.526 55.302) (width 0.7) (layer B.Cu) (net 9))
 (segment (start 90.526 55.302) (end 98.198 55.302) (width 0.7) (layer B.Cu) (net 9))
 (segment (start 98.198 55.302) (end 102.84 59.944) (width 0.7) (layer B.Cu) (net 9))
 (segment (start 102.84 59.944) (end 103.632 59.944) (width 0.7) (layer B.Cu) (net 9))
 (segment (start 78.994 55.372) (end 51.228 55.372) (width 0.7) (layer B.Cu) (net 2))
 (segment (start 51.228 55.372) (end 39.2 67.4) (width 0.7) (layer B.Cu) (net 2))
 (segment (start 39.2 67.4) (end 39.2 77.8) (width 0.7) (layer B.Cu) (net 2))
 (segment (start 39.2 77.8) (end 41.918 80.518) (width 0.7) (layer B.Cu) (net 2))
 (segment (start 41.918 80.518) (end 43.18 80.518) (width 0.7) (layer B.Cu) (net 2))
 (segment (start 78.994 55.372) (end 82.296 55.372) (width 0.7) (layer F.Cu) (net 2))
 (segment (start 82.296 55.372) (end 87.376 60.452) (width 0.7) (layer F.Cu) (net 2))
 (segment (start 67.7 83) (end 67.7 87.512) (width 0.25) (layer F.Cu) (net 12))
 (segment (start 67.7 87.512) (end 68.58 88.392) (width 0.25) (layer F.Cu) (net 12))
 (segment (start 68.58 88.392) (end 68.58 93.472) (width 0.25) (layer F.Cu) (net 12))
 (segment (start 70.24 75.38) (end 76.88 75.38) (width 0.25) (layer F.Cu) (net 13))
 (segment (start 76.88 75.38) (end 86.868 85.368) (width 0.25) (layer F.Cu) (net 13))
 (segment (start 86.868 85.368) (end 86.868 93.472) (width 0.25) (layer F.Cu) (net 13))
 (segment (start 86.868 93.472) (end 85.818 93.472) (width 0.25) (layer F.Cu) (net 13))
 (segment (start 50.292 93.022) (end 50.292 93.472) (width 0.25) (layer F.Cu) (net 14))
 (segment (start 60.08 83) (end 60.08 83.684) (width 0.25) (layer F.Cu) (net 14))
 (segment (start 60.08 83.684) (end 55.118 88.646) (width 0.25) (layer F.Cu) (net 14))
 (segment (start 55.118 88.646) (end 51.308 88.646) (width 0.25) (layer F.Cu) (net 14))
 (segment (start 51.308 88.646) (end 50.292 89.662) (width 0.25) (layer F.Cu) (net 14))
 (segment (start 50.292 89.662) (end 50.292 93.022) (width 0.25) (layer F.Cu) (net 14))
 (segment (start 50.292 93.022) (end 50.292 93.472) (width 0.25) (layer F.Cu) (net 14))
 (segment (start 108.204 93.296) (end 108.204 93.472) (width 0.25) (layer F.Cu) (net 11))
 (segment (start 116.5 85) (end 115.152 85) (width 0.25) (layer F.Cu) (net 11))
 (segment (start 115.152 85) (end 110.998 89.154) (width 0.25) (layer F.Cu) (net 11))
 (segment (start 110.998 89.154) (end 110.236 89.154) (width 0.25) (layer F.Cu) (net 11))
 (segment (start 110.236 89.154) (end 108.204 91.186) (width 0.25) (layer F.Cu) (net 11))
 (segment (start 108.204 91.186) (end 108.204 93.296) (width 0.25) (layer F.Cu) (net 11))
 (segment (start 108.204 93.472) (end 108.204 93.296) (width 0.25) (layer F.Cu) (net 11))
 (segment (start 92 84) (end 95.4 87.4) (width 0.25) (layer F.Cu) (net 17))
 (segment (start 95.4 87.4) (end 111.56 87.4) (width 0.25) (layer F.Cu) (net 17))
 (segment (start 111.56 87.4) (end 116.5 82.46) (width 0.25) (layer F.Cu) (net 17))
 (segment (start 92 76.38) (end 81.88 76.38) (width 0.7) (layer B.Cu) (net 10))
 (segment (start 103.632 54.944) (end 106.444 54.944) (width 0.7) (layer F.Cu) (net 10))
 (segment (start 106.444 54.944) (end 107 55.5) (width 0.7) (layer F.Cu) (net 10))
 (segment (start 107 55.5) (end 107 67.5) (width 0.7) (layer F.Cu) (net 10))
 (segment (start 92.476 56.752) (end 101.824 56.752) (width 0.7) (layer F.Cu) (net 10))
 (segment (start 101.824 56.752) (end 103.632 54.944) (width 0.7) (layer F.Cu) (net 10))
 (segment (start 81.88 76.38) (end 79.26 79) (width 0.7) (layer B.Cu) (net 10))
 (segment (start 79.26 79) (end 58.62 79) (width 0.7) (layer B.Cu) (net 10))
 (segment (start 58.62 79) (end 55 75.38) (width 0.7) (layer B.Cu) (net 10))
 (segment (start 81.88 76.38) (end 75.5 70) (width 0.7) (layer B.Cu) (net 10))
 (segment (start 75.5 70) (end 75.5 62.5) (width 0.7) (layer B.Cu) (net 10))
 (segment (start 75.5 62.5) (end 71.5 58.5) (width 0.7) (layer B.Cu) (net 10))
 (segment (start 71.5 58.5) (end 57.88 58.5) (width 0.7) (layer B.Cu) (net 10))
 (segment (start 57.88 58.5) (end 55 61.38) (width 0.7) (layer B.Cu) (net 10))
 (segment (start 107 67.5) (end 103 71.5) (width 0.7) (layer B.Cu) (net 10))
 (segment (start 103 71.5) (end 96.88 71.5) (width 0.7) (layer B.Cu) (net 10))
 (segment (start 96.88 71.5) (end 92 76.38) (width 0.7) (layer B.Cu) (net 10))
 (segment (start 107 67.5) (end 112.92 67.5) (width 0.7) (layer B.Cu) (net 10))
 (segment (start 112.92 67.5) (end 115 65.42) (width 0.7) (layer B.Cu) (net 10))
 (segment (start 52.4 70.6) (end 54 69) (width 0.25) (layer F.Cu) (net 3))
 (segment (start 54 69) (end 55 69) (width 0.25) (layer F.Cu) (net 3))
 (segment (start 52.6 73) (end 52.6 70.8) (width 0.25) (layer B.Cu) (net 3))
 (segment (start 52.6 70.8) (end 52.4 70.6) (width 0.25) (layer B.Cu) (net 3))
 (segment (start 43.18 76.518) (end 41.098 78.6) (width 0.25) (layer F.Cu) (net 3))
 (segment (start 41.098 78.6) (end 41.098 81.702) (width 0.25) (layer F.Cu) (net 3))
 (segment (start 41.098 81.702) (end 42.796 83.4) (width 0.25) (layer F.Cu) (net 3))
 (segment (start 42.796 83.4) (end 44.8 83.4) (width 0.25) (layer F.Cu) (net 3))
 (segment (start 44.8 83.4) (end 52.6 75.6) (width 0.25) (layer F.Cu) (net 3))
 (segment (start 52.6 75.6) (end 52.6 73) (width 0.25) (layer F.Cu) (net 3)) (via (at 52.4 70.6) (size 0.8) (layers F.Cu B.Cu) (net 3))
 (via (at 52.6 73) (size 0.8) (layers F.Cu B.Cu) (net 3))
 (segment (start 43.18 74.518) (end 40.4 71.738) (width 0.25) (layer F.Cu) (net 4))
 (segment (start 40.4 71.738) (end 40.4 67.7636) (width 0.25) (layer F.Cu) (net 4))
 (segment (start 40.4 67.7636) (end 43.5636 64.6) (width 0.25) (layer F.Cu) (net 4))
 (segment (start 43.5636 64.6) (end 64.48 64.6) (width 0.25) (layer F.Cu) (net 4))
 (segment (start 64.48 64.6) (end 67.7 61.38) (width 0.25) (layer F.Cu) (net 4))
 (segment (start 43.18 72.518) (end 41.162 70.5) (width 0.25) (layer F.Cu) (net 5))
 (segment (start 41.162 70.5) (end 41.162 67.638) (width 0.25) (layer F.Cu) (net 5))
 (segment (start 41.162 67.638) (end 43.6 65.2) (width 0.25) (layer F.Cu) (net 5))
 (segment (start 43.6 65.2) (end 61.36 65.2) (width 0.25) (layer F.Cu) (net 5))
 (segment (start 61.36 65.2) (end 65.16 69) (width 0.25) (layer F.Cu) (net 5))
 (segment (start 45.18 76.518) (end 46.682 76.518) (width 0.25) (layer F.Cu) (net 6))
 (segment (start 46.682 76.518) (end 51.25 71.95) (width 0.25) (layer F.Cu) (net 6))
 (segment (start 51.25 71.95) (end 59.67 71.95) (width 0.25) (layer F.Cu) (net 6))
 (segment (start 59.67 71.95) (end 62.62 69) (width 0.25) (layer F.Cu) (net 6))
 (segment (start 45.18 74.518) (end 47.982 74.518) (width 0.25) (layer F.Cu) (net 7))
 (segment (start 47.982 74.518) (end 51 71.5) (width 0.25) (layer F.Cu) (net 7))
 (segment (start 51 71.5) (end 55.04 71.5) (width 0.25) (layer F.Cu) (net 7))
 (segment (start 55.04 71.5) (end 57.54 69) (width 0.25) (layer F.Cu) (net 7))
 (segment (start 62 63.875) (end 62.665 63.875) (width 0.25) (layer F.Cu) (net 8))
 (segment (start 62.665 63.875) (end 65.16 61.38) (width 0.25) (layer F.Cu) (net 8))
 (segment (start 59.8 65.925) (end 61.85 63.875) (width 0.25) (layer B.Cu) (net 8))
 (segment (start 61.85 63.875) (end 62 63.875) (width 0.25) (layer B.Cu) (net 8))
 (segment (start 45.18 72.518) (end 52.048 65.65) (width 0.25) (layer F.Cu) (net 8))
 (segment (start 52.048 65.65) (end 59.525 65.65) (width 0.25) (layer F.Cu) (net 8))
 (segment (start 59.525 65.65) (end 59.8 65.925) (width 0.25) (layer F.Cu) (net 8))
 (via (at 62 63.875) (size 0.8) (layers F.Cu B.Cu) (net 8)) (via (at 59.8 65.925) (size 0.8) (layers F.Cu B.Cu) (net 8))
 (segment (start 115 70.5) (end 115 72.2) (width 0.25) (layer F.Cu) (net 15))
 (segment (start 115 72.2) (end 107.2 80) (width 0.25) (layer F.Cu) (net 15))
 (segment (start 107.2 80) (end 98.54 80) (width 0.25) (layer F.Cu) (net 15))
 (segment (start 98.54 80) (end 94.54 84) (width 0.25) (layer F.Cu) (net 15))
 (segment (start 65.16 75.38) (end 57.54 83) (width 0.25) (layer F.Cu) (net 16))
 (segment (start 65.16 75.38) (end 65.16 83) (width 0.25) (layer F.Cu) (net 16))
 (segment (start 66.5 73) (end 66.5 74.04) (width 0.25) (layer F.Cu) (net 16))
 (segment (start 66.5 74.04) (end 65.16 75.38) (width 0.25) (layer F.Cu) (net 16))
 (segment (start 73 73) (end 66.5 73) (width 0.25) (layer B.Cu) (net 16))
 (segment (start 115 67.96) (end 109.96 73) (width 0.25) (layer F.Cu) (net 16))
 (segment (start 109.96 73) (end 73 73) (width 0.25) (layer F.Cu) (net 16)) (via (at 66.5 73) (size 0.8) (layers F.Cu B.Cu) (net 16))
 (via (at 73 73) (size 0.8) (layers F.Cu B.Cu) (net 16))
 (segment (start 67.7 75.38) (end 67.7 75.3) (width 0.25) (layer F.Cu) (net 18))
 (segment (start 67.7 75.3) (end 73 70) (width 0.25) (layer F.Cu) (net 18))
 (segment (start 73 70) (end 73 64.14) (width 0.25) (layer F.Cu) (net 18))
 (segment (start 73 64.14) (end 70.24 61.38) (width 0.25) (layer F.Cu) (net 18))
 (segment (start 55 72.8) (end 53.05 74.75) (width 0.25) (layer F.Cu) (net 19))
 (segment (start 53.05 74.75) (end 53.05 76.15) (width 0.25) (layer F.Cu) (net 19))
 (segment (start 53.05 76.15) (end 53 76.2) (width 0.25) (layer F.Cu) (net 19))
 (segment (start 53 76.2) (end 53 81) (width 0.25) (layer F.Cu) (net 19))
 (segment (start 53 81) (end 55 83) (width 0.25) (layer F.Cu) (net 19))
 (segment (start 60.08 69) (end 56.28 72.8) (width 0.25) (layer B.Cu) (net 19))
 (segment (start 56.28 72.8) (end 55 72.8) (width 0.25) (layer B.Cu) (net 19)) (via (at 55 72.8) (size 0.8) (layers F.Cu B.Cu) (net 19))
 (segment (start 64.4 78) (end 64.4 81.22) (width 0.25) (layer F.Cu) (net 20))
 (segment (start 64.4 81.22) (end 62.62 83) (width 0.25) (layer F.Cu) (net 20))
 (segment (start 67.7 69) (end 67.7 71.1) (width 0.25) (layer B.Cu) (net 20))
 (segment (start 67.7 71.1) (end 68.8 72.2) (width 0.25) (layer B.Cu) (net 20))
 (segment (start 68.8 72.2) (end 73.4 72.2) (width 0.25) (layer B.Cu) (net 20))
 (segment (start 73.4 72.2) (end 74.2 73) (width 0.25) (layer B.Cu) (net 20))
 (segment (start 74.2 73) (end 74.2 76) (width 0.25) (layer B.Cu) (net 20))
 (segment (start 74.2 76) (end 72.2 78) (width 0.25) (layer B.Cu) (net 20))
 (segment (start 72.2 78) (end 64.4 78) (width 0.25) (layer B.Cu) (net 20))
 (segment (start 67.7 69) (end 68 69) (width 0.25) (layer F.Cu) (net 20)) (via (at 64.4 78) (size 0.8) (layers F.Cu B.Cu) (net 20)))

